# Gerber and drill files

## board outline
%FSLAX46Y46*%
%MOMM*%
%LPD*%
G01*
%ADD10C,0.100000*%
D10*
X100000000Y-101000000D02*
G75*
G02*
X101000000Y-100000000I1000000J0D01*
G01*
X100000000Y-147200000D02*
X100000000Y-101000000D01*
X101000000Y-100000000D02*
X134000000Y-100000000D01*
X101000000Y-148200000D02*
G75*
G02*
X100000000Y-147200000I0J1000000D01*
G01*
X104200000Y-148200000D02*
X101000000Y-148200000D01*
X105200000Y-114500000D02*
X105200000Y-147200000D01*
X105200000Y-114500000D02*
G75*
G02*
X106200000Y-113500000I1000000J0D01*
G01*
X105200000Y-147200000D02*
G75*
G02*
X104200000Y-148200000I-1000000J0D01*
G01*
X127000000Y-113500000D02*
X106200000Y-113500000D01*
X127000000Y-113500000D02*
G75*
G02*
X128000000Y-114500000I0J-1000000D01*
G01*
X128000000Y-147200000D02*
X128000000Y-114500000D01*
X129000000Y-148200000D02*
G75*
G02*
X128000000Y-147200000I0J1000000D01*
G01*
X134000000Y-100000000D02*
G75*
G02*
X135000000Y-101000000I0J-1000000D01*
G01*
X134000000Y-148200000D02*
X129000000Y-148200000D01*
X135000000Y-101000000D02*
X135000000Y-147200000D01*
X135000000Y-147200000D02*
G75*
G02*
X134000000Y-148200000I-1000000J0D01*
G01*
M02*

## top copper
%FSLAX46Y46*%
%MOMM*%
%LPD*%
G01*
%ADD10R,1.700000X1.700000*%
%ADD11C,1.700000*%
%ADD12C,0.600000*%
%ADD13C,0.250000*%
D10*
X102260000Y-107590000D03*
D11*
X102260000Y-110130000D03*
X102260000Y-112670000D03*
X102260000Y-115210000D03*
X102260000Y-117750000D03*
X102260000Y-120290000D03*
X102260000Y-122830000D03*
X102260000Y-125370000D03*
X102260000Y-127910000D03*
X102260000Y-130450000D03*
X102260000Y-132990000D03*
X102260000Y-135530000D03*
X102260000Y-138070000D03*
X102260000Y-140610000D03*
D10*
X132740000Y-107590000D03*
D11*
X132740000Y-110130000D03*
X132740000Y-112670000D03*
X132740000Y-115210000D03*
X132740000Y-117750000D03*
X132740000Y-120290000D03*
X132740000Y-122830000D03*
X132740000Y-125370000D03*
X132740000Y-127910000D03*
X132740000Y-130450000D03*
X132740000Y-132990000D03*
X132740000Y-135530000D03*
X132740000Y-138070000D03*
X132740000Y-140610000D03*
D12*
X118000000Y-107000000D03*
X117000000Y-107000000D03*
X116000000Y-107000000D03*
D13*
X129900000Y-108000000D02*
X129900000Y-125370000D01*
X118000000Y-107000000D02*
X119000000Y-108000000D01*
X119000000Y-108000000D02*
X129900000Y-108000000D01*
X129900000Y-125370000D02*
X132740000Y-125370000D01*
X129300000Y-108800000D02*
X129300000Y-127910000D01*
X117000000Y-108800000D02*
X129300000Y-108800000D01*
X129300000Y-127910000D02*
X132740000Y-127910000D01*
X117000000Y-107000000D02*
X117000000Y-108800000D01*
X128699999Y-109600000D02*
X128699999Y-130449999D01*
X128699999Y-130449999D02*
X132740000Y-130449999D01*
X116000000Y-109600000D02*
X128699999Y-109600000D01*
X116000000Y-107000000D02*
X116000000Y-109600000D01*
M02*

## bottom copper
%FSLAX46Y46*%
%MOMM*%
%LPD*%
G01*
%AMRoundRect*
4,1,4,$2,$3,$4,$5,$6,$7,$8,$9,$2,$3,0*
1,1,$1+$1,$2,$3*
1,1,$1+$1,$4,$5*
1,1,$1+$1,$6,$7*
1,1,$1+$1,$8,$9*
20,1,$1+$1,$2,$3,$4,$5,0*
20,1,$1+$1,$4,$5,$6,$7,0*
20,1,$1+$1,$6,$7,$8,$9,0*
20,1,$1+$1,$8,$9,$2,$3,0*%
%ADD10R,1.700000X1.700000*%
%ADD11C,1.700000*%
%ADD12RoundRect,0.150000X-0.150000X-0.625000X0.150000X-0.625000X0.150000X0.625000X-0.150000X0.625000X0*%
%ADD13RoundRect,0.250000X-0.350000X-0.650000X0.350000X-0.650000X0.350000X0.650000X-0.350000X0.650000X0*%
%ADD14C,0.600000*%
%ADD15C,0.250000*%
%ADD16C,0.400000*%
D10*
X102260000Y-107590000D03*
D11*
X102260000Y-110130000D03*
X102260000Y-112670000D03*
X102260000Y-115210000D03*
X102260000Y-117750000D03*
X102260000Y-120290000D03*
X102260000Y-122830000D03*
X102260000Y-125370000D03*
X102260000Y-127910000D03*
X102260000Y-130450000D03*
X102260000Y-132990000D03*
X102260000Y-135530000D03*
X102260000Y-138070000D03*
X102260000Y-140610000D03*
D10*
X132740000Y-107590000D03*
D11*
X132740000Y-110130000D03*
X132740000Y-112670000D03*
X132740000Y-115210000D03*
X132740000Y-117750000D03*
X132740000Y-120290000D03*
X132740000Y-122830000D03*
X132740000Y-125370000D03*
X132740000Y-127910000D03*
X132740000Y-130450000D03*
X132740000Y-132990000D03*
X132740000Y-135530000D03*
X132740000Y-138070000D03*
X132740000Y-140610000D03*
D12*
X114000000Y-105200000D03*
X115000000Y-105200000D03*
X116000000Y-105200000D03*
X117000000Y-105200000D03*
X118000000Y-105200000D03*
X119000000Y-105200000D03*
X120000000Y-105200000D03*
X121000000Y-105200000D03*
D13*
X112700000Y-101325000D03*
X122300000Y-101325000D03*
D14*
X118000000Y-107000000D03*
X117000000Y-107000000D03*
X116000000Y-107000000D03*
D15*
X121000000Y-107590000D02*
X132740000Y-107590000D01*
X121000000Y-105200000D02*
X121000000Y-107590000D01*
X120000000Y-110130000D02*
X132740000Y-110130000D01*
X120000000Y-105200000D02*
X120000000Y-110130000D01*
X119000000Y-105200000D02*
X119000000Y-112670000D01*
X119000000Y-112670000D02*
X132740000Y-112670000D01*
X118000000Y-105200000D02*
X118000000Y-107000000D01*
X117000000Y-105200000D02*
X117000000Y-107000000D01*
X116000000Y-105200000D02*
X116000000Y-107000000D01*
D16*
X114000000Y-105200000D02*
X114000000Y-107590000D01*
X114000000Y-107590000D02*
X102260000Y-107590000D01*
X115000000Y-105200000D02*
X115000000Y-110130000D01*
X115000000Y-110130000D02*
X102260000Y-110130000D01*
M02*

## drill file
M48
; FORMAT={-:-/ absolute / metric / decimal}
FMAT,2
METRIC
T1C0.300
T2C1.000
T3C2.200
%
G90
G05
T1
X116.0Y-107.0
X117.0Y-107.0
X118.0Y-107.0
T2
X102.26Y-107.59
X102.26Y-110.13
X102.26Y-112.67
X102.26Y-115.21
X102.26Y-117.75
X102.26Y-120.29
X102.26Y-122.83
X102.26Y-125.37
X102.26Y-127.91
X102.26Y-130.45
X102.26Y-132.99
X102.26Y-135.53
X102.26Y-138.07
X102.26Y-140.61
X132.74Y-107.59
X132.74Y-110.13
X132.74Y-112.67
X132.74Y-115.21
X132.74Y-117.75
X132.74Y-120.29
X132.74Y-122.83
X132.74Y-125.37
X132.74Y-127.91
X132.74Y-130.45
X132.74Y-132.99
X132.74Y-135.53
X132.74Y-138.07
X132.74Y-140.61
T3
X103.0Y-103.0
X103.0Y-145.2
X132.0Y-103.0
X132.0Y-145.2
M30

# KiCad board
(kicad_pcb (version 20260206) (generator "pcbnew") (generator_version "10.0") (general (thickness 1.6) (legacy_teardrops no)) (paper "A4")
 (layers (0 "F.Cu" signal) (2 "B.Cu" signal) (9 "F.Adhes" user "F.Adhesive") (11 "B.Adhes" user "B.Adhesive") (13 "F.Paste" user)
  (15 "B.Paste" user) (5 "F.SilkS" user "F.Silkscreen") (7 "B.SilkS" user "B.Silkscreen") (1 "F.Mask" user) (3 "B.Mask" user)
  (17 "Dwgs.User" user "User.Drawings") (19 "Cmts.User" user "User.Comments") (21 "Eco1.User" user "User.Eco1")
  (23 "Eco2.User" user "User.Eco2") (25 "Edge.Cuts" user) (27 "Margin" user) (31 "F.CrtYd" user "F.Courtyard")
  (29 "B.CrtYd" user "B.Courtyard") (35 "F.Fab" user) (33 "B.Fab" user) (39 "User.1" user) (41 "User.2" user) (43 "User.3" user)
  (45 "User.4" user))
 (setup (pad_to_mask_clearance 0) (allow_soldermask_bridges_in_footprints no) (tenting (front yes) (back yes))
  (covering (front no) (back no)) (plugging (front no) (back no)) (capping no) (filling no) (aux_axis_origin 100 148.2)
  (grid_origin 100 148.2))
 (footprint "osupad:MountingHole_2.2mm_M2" (layer "F.Cu") (at 132 145.2)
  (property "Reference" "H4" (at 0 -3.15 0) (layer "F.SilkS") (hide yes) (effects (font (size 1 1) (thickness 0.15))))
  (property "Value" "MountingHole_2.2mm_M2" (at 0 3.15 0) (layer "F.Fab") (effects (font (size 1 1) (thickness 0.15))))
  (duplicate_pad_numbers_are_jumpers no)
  (pad "" np_thru_hole circle (at 0 0) (size 2.2 2.2) (drill 2.2) (layers "*.Cu" "*.Mask")))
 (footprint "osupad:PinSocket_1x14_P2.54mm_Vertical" (layer "F.Cu") (at 102.26 107.59)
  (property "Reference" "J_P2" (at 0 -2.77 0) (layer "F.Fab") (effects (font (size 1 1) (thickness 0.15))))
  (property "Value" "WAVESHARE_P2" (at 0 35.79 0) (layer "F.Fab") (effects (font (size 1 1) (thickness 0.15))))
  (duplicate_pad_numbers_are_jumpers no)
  (pad "1" thru_hole rect (at 0 0) (size 1.7 1.7) (drill 1) (layers "*.Cu" "*.Mask") (remove_unused_layers no) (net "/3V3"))
  (pad "2" thru_hole circle (at 0 2.54) (size 1.7 1.7) (drill 1) (layers "*.Cu" "*.Mask") (remove_unused_layers no) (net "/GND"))
  (pad "3" thru_hole circle (at 0 5.08) (size 1.7 1.7) (drill 1) (layers "*.Cu" "*.Mask") (remove_unused_layers no)
   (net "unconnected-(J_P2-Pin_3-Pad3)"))
  (pad "4" thru_hole circle (at 0 7.62) (size 1.7 1.7) (drill 1) (layers "*.Cu" "*.Mask") (remove_unused_layers no)
   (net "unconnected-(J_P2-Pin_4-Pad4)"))
  (pad "5" thru_hole circle (at 0 10.16) (size 1.7 1.7) (drill 1) (layers "*.Cu" "*.Mask") (remove_unused_layers no)
   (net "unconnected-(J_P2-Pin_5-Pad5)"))
  (pad "6" thru_hole circle (at 0 12.7) (size 1.7 1.7) (drill 1) (layers "*.Cu" "*.Mask") (remove_unused_layers no)
   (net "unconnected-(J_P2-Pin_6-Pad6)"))
  (pad "7" thru_hole circle (at 0 15.24) (size 1.7 1.7) (drill 1) (layers "*.Cu" "*.Mask") (remove_unused_layers no)
   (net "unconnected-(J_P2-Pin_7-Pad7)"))
  (pad "8" thru_hole circle (at 0 17.78) (size 1.7 1.7) (drill 1) (layers "*.Cu" "*.Mask") (remove_unused_layers no)
   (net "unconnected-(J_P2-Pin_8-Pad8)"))
  (pad "9" thru_hole circle (at 0 20.32) (size 1.7 1.7) (drill 1) (layers "*.Cu" "*.Mask") (remove_unused_layers no)
   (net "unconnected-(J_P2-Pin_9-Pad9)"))
  (pad "10" thru_hole circle (at 0 22.86) (size 1.7 1.7) (drill 1) (layers "*.Cu" "*.Mask") (remove_unused_layers no)
   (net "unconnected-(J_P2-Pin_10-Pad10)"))
  (pad "11" thru_hole circle (at 0 25.4) (size 1.7 1.7) (drill 1) (layers "*.Cu" "*.Mask") (remove_unused_layers no)
   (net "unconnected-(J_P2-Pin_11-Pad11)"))
  (pad "12" thru_hole circle (at 0 27.94) (size 1.7 1.7) (drill 1) (layers "*.Cu" "*.Mask") (remove_unused_layers no)
   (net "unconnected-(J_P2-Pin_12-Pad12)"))
  (pad "13" thru_hole circle (at 0 30.48) (size 1.7 1.7) (drill 1) (layers "*.Cu" "*.Mask") (remove_unused_layers no)
   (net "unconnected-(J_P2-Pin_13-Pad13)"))
  (pad "14" thru_hole circle (at 0 33.02) (size 1.7 1.7) (drill 1) (layers "*.Cu" "*.Mask") (remove_unused_layers no)
   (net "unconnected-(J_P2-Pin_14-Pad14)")))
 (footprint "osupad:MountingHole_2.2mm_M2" (layer "F.Cu") (at 132 103)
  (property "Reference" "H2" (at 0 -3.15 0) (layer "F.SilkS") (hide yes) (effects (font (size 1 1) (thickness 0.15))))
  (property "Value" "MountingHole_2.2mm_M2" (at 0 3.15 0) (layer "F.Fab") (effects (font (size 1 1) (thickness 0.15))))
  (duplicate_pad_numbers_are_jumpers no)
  (pad "" np_thru_hole circle (at 0 0) (size 2.2 2.2) (drill 2.2) (layers "*.Cu" "*.Mask")))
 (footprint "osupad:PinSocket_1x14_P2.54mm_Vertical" (layer "F.Cu") (at 132.74 107.59)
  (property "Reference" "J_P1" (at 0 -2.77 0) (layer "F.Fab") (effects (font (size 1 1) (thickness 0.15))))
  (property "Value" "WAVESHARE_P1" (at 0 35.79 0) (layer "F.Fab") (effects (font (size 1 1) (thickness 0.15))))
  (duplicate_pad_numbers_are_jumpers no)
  (pad "1" thru_hole rect (at 0 0) (size 1.7 1.7) (drill 1) (layers "*.Cu" "*.Mask") (remove_unused_layers no) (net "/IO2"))
  (pad "2" thru_hole circle (at 0 2.54) (size 1.7 1.7) (drill 1) (layers "*.Cu" "*.Mask") (remove_unused_layers no) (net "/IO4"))
  (pad "3" thru_hole circle (at 0 5.08) (size 1.7 1.7) (drill 1) (layers "*.Cu" "*.Mask") (remove_unused_layers no) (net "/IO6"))
  (pad "4" thru_hole circle (at 0 7.62) (size 1.7 1.7) (drill 1) (layers "*.Cu" "*.Mask") (remove_unused_layers no)
   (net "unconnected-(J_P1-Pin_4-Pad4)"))
  (pad "5" thru_hole circle (at 0 10.16) (size 1.7 1.7) (drill 1) (layers "*.Cu" "*.Mask") (remove_unused_layers no)
   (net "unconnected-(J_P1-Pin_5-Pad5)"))
  (pad "6" thru_hole circle (at 0 12.7) (size 1.7 1.7) (drill 1) (layers "*.Cu" "*.Mask") (remove_unused_layers no)
   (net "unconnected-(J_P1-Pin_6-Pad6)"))
  (pad "7" thru_hole circle (at 0 15.24) (size 1.7 1.7) (drill 1) (layers "*.Cu" "*.Mask") (remove_unused_layers no)
   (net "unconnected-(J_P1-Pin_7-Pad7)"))
  (pad "8" thru_hole circle (at 0 17.78) (size 1.7 1.7) (drill 1) (layers "*.Cu" "*.Mask") (remove_unused_layers no) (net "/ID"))
  (pad "9" thru_hole circle (at 0 20.32) (size 1.7 1.7) (drill 1) (layers "*.Cu" "*.Mask") (remove_unused_layers no) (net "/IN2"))
  (pad "10" thru_hole circle (at 0 22.86) (size 1.7 1.7) (drill 1) (layers "*.Cu" "*.Mask") (remove_unused_layers no) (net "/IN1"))
  (pad "11" thru_hole circle (at 0 25.4) (size 1.7 1.7) (drill 1) (layers "*.Cu" "*.Mask") (remove_unused_layers no)
   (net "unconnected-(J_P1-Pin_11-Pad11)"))
  (pad "12" thru_hole circle (at 0 27.94) (size 1.7 1.7) (drill 1) (layers "*.Cu" "*.Mask") (remove_unused_layers no)
   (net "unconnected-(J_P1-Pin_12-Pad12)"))
  (pad "13" thru_hole circle (at 0 30.48) (size 1.7 1.7) (drill 1) (layers "*.Cu" "*.Mask") (remove_unused_layers no)
   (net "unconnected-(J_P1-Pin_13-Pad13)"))
  (pad "14" thru_hole circle (at 0 33.02) (size 1.7 1.7) (drill 1) (layers "*.Cu" "*.Mask") (remove_unused_layers no)
   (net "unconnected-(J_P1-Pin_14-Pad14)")))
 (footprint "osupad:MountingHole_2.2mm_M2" (layer "F.Cu") (at 103 145.2)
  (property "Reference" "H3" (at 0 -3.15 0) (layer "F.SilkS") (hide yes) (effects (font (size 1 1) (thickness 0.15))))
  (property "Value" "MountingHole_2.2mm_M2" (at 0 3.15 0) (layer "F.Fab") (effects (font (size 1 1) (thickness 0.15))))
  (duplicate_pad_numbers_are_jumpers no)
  (pad "" np_thru_hole circle (at 0 0) (size 2.2 2.2) (drill 2.2) (layers "*.Cu" "*.Mask")))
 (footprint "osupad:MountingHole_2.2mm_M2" (layer "F.Cu") (at 103 103)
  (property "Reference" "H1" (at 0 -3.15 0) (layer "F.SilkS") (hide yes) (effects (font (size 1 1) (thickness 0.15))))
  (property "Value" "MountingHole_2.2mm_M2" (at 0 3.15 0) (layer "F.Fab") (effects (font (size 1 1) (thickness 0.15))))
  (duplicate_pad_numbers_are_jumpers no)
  (pad "" np_thru_hole circle (at 0 0) (size 2.2 2.2) (drill 2.2) (layers "*.Cu" "*.Mask")))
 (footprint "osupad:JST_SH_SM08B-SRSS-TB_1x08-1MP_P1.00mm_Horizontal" (layer "B.Cu") (at 117.5 103.2)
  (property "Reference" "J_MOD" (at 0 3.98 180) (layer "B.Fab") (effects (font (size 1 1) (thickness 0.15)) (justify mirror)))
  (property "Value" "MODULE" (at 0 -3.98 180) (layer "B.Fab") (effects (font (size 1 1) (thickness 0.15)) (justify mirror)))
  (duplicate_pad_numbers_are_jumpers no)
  (pad "1" smd roundrect (at -3.5 2) (size 0.6 1.55) (layers "B.Cu" "B.Mask" "B.Paste") (roundrect_rratio 0.25) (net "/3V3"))
  (pad "2" smd roundrect (at -2.5 2) (size 0.6 1.55) (layers "B.Cu" "B.Mask" "B.Paste") (roundrect_rratio 0.25) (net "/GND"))
  (pad "3" smd roundrect (at -1.5 2) (size 0.6 1.55) (layers "B.Cu" "B.Mask" "B.Paste") (roundrect_rratio 0.25) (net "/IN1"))
  (pad "4" smd roundrect (at -0.5 2) (size 0.6 1.55) (layers "B.Cu" "B.Mask" "B.Paste") (roundrect_rratio 0.25) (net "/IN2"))
  (pad "5" smd roundrect (at 0.5 2) (size 0.6 1.55) (layers "B.Cu" "B.Mask" "B.Paste") (roundrect_rratio 0.25) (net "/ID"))
  (pad "6" smd roundrect (at 1.5 2) (size 0.6 1.55) (layers "B.Cu" "B.Mask" "B.Paste") (roundrect_rratio 0.25) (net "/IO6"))
  (pad "7" smd roundrect (at 2.5 2) (size 0.6 1.55) (layers "B.Cu" "B.Mask" "B.Paste") (roundrect_rratio 0.25) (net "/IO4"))
  (pad "8" smd roundrect (at 3.5 2) (size 0.6 1.55) (layers "B.Cu" "B.Mask" "B.Paste") (roundrect_rratio 0.25) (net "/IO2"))
  (pad "MP" smd roundrect (at -4.8 -1.875) (size 1.2 1.8) (layers "B.Cu" "B.Mask" "B.Paste") (roundrect_rratio 0.208333))
  (pad "MP" smd roundrect (at 4.8 -1.875) (size 1.2 1.8) (layers "B.Cu" "B.Mask" "B.Paste") (roundrect_rratio 0.208333)))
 (gr_arc (start 100 101) (mid 100.292893 100.292893) (end 101 100) (stroke (width 0.1) (type default)) (layer "Edge.Cuts"))
 (gr_line (start 100 147.2) (end 100 101) (stroke (width 0.1) (type default)) (layer "Edge.Cuts"))
 (gr_line (start 101 100) (end 134 100) (stroke (width 0.1) (type default)) (layer "Edge.Cuts"))
 (gr_arc (start 101 148.2) (mid 100.292893 147.907106) (end 100 147.2) (stroke (width 0.1) (type default)) (layer "Edge.Cuts"))
 (gr_line (start 104.2 148.2) (end 101 148.2) (stroke (width 0.1) (type default)) (layer "Edge.Cuts"))
 (gr_line (start 105.2 114.5) (end 105.2 147.2) (stroke (width 0.1) (type default)) (layer "Edge.Cuts"))
 (gr_arc (start 105.2 114.5) (mid 105.492893 113.792893) (end 106.2 113.5) (stroke (width 0.1) (type default)) (layer "Edge.Cuts"))
 (gr_arc (start 105.2 147.2) (mid 104.907106 147.907106) (end 104.2 148.2) (stroke (width 0.1) (type default)) (layer "Edge.Cuts"))
 (gr_line (start 127 113.5) (end 106.2 113.5) (stroke (width 0.1) (type default)) (layer "Edge.Cuts"))
 (gr_arc (start 127 113.5) (mid 127.707107 113.792893) (end 128 114.5) (stroke (width 0.1) (type default)) (layer "Edge.Cuts"))
 (gr_line (start 128 147.2) (end 128 114.5) (stroke (width 0.1) (type default)) (layer "Edge.Cuts"))
 (gr_arc (start 129 148.2) (mid 128.292893 147.907106) (end 128 147.2) (stroke (width 0.1) (type default)) (layer "Edge.Cuts"))
 (gr_arc (start 134 100) (mid 134.707106 100.292893) (end 135 101) (stroke (width 0.1) (type default)) (layer "Edge.Cuts"))
 (gr_line (start 134 148.2) (end 129 148.2) (stroke (width 0.1) (type default)) (layer "Edge.Cuts"))
 (gr_line (start 135 101) (end 135 147.2) (stroke (width 0.1) (type default)) (layer "Edge.Cuts"))
 (gr_arc (start 135 147.2) (mid 134.707106 147.907106) (end 134 148.2) (stroke (width 0.1) (type default)) (layer "Edge.Cuts"))
 (segment (start 121 107.59) (end 132.74 107.59) (width 0.25) (layer "B.Cu") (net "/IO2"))
 (segment (start 121 105.2) (end 121 107.59) (width 0.25) (layer "B.Cu") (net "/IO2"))
 (segment (start 120 110.13) (end 132.74 110.13) (width 0.25) (layer "B.Cu") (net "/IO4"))
 (segment (start 120 105.2) (end 120 110.13) (width 0.25) (layer "B.Cu") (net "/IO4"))
 (segment (start 119 105.2) (end 119 112.67) (width 0.25) (layer "B.Cu") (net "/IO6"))
 (segment (start 119 112.67) (end 132.74 112.67) (width 0.25) (layer "B.Cu") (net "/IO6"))
 (segment (start 129.9 108) (end 129.9 125.37) (width 0.25) (layer "F.Cu") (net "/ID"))
 (segment (start 118 107) (end 119 108) (width 0.25) (layer "F.Cu") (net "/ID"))
 (segment (start 119 108) (end 129.9 108) (width 0.25) (layer "F.Cu") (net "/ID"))
 (segment (start 129.9 125.37) (end 132.74 125.37) (width 0.25) (layer "F.Cu") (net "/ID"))
 (via (at 118 107) (size 0.6) (drill 0.3) (layers "F.Cu" "B.Cu") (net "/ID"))
 (segment (start 118 105.2) (end 118 107) (width 0.25) (layer "B.Cu") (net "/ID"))
 (segment (start 129.3 108.8) (end 129.3 127.91) (width 0.25) (layer "F.Cu") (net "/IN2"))
 (segment (start 117 108.8) (end 129.3 108.8) (width 0.25) (layer "F.Cu") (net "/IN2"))
 (segment (start 129.3 127.91) (end 132.74 127.91) (width 0.25) (layer "F.Cu") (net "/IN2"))
 (segment (start 117 107) (end 117 108.8) (width 0.25) (layer "F.Cu") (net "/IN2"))
 (via (at 117 107) (size 0.6) (drill 0.3) (layers "F.Cu" "B.Cu") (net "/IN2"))
 (segment (start 117 105.2) (end 117 107) (width 0.25) (layer "B.Cu") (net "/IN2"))
 (segment (start 128.699999 109.6) (end 128.699999 130.449999) (width 0.25) (layer "F.Cu") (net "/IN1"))
 (segment (start 128.699999 130.449999) (end 132.74 130.449999) (width 0.25) (layer "F.Cu") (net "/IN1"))
 (segment (start 116 109.6) (end 128.699999 109.6) (width 0.25) (layer "F.Cu") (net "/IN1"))
 (segment (start 116 107) (end 116 109.6) (width 0.25) (layer "F.Cu") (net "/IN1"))
 (via (at 116 107) (size 0.6) (drill 0.3) (layers "F.Cu" "B.Cu") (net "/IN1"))
 (segment (start 116 105.2) (end 116 107) (width 0.25) (layer "B.Cu") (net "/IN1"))
 (segment (start 114 105.2) (end 114 107.59) (width 0.4) (layer "B.Cu") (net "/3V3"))
 (segment (start 114 107.59) (end 102.26 107.59) (width 0.4) (layer "B.Cu") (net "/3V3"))
 (segment (start 115 105.2) (end 115 110.13) (width 0.4) (layer "B.Cu") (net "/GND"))
 (segment (start 115 110.13) (end 102.26 110.13) (width 0.4) (layer "B.Cu") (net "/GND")))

